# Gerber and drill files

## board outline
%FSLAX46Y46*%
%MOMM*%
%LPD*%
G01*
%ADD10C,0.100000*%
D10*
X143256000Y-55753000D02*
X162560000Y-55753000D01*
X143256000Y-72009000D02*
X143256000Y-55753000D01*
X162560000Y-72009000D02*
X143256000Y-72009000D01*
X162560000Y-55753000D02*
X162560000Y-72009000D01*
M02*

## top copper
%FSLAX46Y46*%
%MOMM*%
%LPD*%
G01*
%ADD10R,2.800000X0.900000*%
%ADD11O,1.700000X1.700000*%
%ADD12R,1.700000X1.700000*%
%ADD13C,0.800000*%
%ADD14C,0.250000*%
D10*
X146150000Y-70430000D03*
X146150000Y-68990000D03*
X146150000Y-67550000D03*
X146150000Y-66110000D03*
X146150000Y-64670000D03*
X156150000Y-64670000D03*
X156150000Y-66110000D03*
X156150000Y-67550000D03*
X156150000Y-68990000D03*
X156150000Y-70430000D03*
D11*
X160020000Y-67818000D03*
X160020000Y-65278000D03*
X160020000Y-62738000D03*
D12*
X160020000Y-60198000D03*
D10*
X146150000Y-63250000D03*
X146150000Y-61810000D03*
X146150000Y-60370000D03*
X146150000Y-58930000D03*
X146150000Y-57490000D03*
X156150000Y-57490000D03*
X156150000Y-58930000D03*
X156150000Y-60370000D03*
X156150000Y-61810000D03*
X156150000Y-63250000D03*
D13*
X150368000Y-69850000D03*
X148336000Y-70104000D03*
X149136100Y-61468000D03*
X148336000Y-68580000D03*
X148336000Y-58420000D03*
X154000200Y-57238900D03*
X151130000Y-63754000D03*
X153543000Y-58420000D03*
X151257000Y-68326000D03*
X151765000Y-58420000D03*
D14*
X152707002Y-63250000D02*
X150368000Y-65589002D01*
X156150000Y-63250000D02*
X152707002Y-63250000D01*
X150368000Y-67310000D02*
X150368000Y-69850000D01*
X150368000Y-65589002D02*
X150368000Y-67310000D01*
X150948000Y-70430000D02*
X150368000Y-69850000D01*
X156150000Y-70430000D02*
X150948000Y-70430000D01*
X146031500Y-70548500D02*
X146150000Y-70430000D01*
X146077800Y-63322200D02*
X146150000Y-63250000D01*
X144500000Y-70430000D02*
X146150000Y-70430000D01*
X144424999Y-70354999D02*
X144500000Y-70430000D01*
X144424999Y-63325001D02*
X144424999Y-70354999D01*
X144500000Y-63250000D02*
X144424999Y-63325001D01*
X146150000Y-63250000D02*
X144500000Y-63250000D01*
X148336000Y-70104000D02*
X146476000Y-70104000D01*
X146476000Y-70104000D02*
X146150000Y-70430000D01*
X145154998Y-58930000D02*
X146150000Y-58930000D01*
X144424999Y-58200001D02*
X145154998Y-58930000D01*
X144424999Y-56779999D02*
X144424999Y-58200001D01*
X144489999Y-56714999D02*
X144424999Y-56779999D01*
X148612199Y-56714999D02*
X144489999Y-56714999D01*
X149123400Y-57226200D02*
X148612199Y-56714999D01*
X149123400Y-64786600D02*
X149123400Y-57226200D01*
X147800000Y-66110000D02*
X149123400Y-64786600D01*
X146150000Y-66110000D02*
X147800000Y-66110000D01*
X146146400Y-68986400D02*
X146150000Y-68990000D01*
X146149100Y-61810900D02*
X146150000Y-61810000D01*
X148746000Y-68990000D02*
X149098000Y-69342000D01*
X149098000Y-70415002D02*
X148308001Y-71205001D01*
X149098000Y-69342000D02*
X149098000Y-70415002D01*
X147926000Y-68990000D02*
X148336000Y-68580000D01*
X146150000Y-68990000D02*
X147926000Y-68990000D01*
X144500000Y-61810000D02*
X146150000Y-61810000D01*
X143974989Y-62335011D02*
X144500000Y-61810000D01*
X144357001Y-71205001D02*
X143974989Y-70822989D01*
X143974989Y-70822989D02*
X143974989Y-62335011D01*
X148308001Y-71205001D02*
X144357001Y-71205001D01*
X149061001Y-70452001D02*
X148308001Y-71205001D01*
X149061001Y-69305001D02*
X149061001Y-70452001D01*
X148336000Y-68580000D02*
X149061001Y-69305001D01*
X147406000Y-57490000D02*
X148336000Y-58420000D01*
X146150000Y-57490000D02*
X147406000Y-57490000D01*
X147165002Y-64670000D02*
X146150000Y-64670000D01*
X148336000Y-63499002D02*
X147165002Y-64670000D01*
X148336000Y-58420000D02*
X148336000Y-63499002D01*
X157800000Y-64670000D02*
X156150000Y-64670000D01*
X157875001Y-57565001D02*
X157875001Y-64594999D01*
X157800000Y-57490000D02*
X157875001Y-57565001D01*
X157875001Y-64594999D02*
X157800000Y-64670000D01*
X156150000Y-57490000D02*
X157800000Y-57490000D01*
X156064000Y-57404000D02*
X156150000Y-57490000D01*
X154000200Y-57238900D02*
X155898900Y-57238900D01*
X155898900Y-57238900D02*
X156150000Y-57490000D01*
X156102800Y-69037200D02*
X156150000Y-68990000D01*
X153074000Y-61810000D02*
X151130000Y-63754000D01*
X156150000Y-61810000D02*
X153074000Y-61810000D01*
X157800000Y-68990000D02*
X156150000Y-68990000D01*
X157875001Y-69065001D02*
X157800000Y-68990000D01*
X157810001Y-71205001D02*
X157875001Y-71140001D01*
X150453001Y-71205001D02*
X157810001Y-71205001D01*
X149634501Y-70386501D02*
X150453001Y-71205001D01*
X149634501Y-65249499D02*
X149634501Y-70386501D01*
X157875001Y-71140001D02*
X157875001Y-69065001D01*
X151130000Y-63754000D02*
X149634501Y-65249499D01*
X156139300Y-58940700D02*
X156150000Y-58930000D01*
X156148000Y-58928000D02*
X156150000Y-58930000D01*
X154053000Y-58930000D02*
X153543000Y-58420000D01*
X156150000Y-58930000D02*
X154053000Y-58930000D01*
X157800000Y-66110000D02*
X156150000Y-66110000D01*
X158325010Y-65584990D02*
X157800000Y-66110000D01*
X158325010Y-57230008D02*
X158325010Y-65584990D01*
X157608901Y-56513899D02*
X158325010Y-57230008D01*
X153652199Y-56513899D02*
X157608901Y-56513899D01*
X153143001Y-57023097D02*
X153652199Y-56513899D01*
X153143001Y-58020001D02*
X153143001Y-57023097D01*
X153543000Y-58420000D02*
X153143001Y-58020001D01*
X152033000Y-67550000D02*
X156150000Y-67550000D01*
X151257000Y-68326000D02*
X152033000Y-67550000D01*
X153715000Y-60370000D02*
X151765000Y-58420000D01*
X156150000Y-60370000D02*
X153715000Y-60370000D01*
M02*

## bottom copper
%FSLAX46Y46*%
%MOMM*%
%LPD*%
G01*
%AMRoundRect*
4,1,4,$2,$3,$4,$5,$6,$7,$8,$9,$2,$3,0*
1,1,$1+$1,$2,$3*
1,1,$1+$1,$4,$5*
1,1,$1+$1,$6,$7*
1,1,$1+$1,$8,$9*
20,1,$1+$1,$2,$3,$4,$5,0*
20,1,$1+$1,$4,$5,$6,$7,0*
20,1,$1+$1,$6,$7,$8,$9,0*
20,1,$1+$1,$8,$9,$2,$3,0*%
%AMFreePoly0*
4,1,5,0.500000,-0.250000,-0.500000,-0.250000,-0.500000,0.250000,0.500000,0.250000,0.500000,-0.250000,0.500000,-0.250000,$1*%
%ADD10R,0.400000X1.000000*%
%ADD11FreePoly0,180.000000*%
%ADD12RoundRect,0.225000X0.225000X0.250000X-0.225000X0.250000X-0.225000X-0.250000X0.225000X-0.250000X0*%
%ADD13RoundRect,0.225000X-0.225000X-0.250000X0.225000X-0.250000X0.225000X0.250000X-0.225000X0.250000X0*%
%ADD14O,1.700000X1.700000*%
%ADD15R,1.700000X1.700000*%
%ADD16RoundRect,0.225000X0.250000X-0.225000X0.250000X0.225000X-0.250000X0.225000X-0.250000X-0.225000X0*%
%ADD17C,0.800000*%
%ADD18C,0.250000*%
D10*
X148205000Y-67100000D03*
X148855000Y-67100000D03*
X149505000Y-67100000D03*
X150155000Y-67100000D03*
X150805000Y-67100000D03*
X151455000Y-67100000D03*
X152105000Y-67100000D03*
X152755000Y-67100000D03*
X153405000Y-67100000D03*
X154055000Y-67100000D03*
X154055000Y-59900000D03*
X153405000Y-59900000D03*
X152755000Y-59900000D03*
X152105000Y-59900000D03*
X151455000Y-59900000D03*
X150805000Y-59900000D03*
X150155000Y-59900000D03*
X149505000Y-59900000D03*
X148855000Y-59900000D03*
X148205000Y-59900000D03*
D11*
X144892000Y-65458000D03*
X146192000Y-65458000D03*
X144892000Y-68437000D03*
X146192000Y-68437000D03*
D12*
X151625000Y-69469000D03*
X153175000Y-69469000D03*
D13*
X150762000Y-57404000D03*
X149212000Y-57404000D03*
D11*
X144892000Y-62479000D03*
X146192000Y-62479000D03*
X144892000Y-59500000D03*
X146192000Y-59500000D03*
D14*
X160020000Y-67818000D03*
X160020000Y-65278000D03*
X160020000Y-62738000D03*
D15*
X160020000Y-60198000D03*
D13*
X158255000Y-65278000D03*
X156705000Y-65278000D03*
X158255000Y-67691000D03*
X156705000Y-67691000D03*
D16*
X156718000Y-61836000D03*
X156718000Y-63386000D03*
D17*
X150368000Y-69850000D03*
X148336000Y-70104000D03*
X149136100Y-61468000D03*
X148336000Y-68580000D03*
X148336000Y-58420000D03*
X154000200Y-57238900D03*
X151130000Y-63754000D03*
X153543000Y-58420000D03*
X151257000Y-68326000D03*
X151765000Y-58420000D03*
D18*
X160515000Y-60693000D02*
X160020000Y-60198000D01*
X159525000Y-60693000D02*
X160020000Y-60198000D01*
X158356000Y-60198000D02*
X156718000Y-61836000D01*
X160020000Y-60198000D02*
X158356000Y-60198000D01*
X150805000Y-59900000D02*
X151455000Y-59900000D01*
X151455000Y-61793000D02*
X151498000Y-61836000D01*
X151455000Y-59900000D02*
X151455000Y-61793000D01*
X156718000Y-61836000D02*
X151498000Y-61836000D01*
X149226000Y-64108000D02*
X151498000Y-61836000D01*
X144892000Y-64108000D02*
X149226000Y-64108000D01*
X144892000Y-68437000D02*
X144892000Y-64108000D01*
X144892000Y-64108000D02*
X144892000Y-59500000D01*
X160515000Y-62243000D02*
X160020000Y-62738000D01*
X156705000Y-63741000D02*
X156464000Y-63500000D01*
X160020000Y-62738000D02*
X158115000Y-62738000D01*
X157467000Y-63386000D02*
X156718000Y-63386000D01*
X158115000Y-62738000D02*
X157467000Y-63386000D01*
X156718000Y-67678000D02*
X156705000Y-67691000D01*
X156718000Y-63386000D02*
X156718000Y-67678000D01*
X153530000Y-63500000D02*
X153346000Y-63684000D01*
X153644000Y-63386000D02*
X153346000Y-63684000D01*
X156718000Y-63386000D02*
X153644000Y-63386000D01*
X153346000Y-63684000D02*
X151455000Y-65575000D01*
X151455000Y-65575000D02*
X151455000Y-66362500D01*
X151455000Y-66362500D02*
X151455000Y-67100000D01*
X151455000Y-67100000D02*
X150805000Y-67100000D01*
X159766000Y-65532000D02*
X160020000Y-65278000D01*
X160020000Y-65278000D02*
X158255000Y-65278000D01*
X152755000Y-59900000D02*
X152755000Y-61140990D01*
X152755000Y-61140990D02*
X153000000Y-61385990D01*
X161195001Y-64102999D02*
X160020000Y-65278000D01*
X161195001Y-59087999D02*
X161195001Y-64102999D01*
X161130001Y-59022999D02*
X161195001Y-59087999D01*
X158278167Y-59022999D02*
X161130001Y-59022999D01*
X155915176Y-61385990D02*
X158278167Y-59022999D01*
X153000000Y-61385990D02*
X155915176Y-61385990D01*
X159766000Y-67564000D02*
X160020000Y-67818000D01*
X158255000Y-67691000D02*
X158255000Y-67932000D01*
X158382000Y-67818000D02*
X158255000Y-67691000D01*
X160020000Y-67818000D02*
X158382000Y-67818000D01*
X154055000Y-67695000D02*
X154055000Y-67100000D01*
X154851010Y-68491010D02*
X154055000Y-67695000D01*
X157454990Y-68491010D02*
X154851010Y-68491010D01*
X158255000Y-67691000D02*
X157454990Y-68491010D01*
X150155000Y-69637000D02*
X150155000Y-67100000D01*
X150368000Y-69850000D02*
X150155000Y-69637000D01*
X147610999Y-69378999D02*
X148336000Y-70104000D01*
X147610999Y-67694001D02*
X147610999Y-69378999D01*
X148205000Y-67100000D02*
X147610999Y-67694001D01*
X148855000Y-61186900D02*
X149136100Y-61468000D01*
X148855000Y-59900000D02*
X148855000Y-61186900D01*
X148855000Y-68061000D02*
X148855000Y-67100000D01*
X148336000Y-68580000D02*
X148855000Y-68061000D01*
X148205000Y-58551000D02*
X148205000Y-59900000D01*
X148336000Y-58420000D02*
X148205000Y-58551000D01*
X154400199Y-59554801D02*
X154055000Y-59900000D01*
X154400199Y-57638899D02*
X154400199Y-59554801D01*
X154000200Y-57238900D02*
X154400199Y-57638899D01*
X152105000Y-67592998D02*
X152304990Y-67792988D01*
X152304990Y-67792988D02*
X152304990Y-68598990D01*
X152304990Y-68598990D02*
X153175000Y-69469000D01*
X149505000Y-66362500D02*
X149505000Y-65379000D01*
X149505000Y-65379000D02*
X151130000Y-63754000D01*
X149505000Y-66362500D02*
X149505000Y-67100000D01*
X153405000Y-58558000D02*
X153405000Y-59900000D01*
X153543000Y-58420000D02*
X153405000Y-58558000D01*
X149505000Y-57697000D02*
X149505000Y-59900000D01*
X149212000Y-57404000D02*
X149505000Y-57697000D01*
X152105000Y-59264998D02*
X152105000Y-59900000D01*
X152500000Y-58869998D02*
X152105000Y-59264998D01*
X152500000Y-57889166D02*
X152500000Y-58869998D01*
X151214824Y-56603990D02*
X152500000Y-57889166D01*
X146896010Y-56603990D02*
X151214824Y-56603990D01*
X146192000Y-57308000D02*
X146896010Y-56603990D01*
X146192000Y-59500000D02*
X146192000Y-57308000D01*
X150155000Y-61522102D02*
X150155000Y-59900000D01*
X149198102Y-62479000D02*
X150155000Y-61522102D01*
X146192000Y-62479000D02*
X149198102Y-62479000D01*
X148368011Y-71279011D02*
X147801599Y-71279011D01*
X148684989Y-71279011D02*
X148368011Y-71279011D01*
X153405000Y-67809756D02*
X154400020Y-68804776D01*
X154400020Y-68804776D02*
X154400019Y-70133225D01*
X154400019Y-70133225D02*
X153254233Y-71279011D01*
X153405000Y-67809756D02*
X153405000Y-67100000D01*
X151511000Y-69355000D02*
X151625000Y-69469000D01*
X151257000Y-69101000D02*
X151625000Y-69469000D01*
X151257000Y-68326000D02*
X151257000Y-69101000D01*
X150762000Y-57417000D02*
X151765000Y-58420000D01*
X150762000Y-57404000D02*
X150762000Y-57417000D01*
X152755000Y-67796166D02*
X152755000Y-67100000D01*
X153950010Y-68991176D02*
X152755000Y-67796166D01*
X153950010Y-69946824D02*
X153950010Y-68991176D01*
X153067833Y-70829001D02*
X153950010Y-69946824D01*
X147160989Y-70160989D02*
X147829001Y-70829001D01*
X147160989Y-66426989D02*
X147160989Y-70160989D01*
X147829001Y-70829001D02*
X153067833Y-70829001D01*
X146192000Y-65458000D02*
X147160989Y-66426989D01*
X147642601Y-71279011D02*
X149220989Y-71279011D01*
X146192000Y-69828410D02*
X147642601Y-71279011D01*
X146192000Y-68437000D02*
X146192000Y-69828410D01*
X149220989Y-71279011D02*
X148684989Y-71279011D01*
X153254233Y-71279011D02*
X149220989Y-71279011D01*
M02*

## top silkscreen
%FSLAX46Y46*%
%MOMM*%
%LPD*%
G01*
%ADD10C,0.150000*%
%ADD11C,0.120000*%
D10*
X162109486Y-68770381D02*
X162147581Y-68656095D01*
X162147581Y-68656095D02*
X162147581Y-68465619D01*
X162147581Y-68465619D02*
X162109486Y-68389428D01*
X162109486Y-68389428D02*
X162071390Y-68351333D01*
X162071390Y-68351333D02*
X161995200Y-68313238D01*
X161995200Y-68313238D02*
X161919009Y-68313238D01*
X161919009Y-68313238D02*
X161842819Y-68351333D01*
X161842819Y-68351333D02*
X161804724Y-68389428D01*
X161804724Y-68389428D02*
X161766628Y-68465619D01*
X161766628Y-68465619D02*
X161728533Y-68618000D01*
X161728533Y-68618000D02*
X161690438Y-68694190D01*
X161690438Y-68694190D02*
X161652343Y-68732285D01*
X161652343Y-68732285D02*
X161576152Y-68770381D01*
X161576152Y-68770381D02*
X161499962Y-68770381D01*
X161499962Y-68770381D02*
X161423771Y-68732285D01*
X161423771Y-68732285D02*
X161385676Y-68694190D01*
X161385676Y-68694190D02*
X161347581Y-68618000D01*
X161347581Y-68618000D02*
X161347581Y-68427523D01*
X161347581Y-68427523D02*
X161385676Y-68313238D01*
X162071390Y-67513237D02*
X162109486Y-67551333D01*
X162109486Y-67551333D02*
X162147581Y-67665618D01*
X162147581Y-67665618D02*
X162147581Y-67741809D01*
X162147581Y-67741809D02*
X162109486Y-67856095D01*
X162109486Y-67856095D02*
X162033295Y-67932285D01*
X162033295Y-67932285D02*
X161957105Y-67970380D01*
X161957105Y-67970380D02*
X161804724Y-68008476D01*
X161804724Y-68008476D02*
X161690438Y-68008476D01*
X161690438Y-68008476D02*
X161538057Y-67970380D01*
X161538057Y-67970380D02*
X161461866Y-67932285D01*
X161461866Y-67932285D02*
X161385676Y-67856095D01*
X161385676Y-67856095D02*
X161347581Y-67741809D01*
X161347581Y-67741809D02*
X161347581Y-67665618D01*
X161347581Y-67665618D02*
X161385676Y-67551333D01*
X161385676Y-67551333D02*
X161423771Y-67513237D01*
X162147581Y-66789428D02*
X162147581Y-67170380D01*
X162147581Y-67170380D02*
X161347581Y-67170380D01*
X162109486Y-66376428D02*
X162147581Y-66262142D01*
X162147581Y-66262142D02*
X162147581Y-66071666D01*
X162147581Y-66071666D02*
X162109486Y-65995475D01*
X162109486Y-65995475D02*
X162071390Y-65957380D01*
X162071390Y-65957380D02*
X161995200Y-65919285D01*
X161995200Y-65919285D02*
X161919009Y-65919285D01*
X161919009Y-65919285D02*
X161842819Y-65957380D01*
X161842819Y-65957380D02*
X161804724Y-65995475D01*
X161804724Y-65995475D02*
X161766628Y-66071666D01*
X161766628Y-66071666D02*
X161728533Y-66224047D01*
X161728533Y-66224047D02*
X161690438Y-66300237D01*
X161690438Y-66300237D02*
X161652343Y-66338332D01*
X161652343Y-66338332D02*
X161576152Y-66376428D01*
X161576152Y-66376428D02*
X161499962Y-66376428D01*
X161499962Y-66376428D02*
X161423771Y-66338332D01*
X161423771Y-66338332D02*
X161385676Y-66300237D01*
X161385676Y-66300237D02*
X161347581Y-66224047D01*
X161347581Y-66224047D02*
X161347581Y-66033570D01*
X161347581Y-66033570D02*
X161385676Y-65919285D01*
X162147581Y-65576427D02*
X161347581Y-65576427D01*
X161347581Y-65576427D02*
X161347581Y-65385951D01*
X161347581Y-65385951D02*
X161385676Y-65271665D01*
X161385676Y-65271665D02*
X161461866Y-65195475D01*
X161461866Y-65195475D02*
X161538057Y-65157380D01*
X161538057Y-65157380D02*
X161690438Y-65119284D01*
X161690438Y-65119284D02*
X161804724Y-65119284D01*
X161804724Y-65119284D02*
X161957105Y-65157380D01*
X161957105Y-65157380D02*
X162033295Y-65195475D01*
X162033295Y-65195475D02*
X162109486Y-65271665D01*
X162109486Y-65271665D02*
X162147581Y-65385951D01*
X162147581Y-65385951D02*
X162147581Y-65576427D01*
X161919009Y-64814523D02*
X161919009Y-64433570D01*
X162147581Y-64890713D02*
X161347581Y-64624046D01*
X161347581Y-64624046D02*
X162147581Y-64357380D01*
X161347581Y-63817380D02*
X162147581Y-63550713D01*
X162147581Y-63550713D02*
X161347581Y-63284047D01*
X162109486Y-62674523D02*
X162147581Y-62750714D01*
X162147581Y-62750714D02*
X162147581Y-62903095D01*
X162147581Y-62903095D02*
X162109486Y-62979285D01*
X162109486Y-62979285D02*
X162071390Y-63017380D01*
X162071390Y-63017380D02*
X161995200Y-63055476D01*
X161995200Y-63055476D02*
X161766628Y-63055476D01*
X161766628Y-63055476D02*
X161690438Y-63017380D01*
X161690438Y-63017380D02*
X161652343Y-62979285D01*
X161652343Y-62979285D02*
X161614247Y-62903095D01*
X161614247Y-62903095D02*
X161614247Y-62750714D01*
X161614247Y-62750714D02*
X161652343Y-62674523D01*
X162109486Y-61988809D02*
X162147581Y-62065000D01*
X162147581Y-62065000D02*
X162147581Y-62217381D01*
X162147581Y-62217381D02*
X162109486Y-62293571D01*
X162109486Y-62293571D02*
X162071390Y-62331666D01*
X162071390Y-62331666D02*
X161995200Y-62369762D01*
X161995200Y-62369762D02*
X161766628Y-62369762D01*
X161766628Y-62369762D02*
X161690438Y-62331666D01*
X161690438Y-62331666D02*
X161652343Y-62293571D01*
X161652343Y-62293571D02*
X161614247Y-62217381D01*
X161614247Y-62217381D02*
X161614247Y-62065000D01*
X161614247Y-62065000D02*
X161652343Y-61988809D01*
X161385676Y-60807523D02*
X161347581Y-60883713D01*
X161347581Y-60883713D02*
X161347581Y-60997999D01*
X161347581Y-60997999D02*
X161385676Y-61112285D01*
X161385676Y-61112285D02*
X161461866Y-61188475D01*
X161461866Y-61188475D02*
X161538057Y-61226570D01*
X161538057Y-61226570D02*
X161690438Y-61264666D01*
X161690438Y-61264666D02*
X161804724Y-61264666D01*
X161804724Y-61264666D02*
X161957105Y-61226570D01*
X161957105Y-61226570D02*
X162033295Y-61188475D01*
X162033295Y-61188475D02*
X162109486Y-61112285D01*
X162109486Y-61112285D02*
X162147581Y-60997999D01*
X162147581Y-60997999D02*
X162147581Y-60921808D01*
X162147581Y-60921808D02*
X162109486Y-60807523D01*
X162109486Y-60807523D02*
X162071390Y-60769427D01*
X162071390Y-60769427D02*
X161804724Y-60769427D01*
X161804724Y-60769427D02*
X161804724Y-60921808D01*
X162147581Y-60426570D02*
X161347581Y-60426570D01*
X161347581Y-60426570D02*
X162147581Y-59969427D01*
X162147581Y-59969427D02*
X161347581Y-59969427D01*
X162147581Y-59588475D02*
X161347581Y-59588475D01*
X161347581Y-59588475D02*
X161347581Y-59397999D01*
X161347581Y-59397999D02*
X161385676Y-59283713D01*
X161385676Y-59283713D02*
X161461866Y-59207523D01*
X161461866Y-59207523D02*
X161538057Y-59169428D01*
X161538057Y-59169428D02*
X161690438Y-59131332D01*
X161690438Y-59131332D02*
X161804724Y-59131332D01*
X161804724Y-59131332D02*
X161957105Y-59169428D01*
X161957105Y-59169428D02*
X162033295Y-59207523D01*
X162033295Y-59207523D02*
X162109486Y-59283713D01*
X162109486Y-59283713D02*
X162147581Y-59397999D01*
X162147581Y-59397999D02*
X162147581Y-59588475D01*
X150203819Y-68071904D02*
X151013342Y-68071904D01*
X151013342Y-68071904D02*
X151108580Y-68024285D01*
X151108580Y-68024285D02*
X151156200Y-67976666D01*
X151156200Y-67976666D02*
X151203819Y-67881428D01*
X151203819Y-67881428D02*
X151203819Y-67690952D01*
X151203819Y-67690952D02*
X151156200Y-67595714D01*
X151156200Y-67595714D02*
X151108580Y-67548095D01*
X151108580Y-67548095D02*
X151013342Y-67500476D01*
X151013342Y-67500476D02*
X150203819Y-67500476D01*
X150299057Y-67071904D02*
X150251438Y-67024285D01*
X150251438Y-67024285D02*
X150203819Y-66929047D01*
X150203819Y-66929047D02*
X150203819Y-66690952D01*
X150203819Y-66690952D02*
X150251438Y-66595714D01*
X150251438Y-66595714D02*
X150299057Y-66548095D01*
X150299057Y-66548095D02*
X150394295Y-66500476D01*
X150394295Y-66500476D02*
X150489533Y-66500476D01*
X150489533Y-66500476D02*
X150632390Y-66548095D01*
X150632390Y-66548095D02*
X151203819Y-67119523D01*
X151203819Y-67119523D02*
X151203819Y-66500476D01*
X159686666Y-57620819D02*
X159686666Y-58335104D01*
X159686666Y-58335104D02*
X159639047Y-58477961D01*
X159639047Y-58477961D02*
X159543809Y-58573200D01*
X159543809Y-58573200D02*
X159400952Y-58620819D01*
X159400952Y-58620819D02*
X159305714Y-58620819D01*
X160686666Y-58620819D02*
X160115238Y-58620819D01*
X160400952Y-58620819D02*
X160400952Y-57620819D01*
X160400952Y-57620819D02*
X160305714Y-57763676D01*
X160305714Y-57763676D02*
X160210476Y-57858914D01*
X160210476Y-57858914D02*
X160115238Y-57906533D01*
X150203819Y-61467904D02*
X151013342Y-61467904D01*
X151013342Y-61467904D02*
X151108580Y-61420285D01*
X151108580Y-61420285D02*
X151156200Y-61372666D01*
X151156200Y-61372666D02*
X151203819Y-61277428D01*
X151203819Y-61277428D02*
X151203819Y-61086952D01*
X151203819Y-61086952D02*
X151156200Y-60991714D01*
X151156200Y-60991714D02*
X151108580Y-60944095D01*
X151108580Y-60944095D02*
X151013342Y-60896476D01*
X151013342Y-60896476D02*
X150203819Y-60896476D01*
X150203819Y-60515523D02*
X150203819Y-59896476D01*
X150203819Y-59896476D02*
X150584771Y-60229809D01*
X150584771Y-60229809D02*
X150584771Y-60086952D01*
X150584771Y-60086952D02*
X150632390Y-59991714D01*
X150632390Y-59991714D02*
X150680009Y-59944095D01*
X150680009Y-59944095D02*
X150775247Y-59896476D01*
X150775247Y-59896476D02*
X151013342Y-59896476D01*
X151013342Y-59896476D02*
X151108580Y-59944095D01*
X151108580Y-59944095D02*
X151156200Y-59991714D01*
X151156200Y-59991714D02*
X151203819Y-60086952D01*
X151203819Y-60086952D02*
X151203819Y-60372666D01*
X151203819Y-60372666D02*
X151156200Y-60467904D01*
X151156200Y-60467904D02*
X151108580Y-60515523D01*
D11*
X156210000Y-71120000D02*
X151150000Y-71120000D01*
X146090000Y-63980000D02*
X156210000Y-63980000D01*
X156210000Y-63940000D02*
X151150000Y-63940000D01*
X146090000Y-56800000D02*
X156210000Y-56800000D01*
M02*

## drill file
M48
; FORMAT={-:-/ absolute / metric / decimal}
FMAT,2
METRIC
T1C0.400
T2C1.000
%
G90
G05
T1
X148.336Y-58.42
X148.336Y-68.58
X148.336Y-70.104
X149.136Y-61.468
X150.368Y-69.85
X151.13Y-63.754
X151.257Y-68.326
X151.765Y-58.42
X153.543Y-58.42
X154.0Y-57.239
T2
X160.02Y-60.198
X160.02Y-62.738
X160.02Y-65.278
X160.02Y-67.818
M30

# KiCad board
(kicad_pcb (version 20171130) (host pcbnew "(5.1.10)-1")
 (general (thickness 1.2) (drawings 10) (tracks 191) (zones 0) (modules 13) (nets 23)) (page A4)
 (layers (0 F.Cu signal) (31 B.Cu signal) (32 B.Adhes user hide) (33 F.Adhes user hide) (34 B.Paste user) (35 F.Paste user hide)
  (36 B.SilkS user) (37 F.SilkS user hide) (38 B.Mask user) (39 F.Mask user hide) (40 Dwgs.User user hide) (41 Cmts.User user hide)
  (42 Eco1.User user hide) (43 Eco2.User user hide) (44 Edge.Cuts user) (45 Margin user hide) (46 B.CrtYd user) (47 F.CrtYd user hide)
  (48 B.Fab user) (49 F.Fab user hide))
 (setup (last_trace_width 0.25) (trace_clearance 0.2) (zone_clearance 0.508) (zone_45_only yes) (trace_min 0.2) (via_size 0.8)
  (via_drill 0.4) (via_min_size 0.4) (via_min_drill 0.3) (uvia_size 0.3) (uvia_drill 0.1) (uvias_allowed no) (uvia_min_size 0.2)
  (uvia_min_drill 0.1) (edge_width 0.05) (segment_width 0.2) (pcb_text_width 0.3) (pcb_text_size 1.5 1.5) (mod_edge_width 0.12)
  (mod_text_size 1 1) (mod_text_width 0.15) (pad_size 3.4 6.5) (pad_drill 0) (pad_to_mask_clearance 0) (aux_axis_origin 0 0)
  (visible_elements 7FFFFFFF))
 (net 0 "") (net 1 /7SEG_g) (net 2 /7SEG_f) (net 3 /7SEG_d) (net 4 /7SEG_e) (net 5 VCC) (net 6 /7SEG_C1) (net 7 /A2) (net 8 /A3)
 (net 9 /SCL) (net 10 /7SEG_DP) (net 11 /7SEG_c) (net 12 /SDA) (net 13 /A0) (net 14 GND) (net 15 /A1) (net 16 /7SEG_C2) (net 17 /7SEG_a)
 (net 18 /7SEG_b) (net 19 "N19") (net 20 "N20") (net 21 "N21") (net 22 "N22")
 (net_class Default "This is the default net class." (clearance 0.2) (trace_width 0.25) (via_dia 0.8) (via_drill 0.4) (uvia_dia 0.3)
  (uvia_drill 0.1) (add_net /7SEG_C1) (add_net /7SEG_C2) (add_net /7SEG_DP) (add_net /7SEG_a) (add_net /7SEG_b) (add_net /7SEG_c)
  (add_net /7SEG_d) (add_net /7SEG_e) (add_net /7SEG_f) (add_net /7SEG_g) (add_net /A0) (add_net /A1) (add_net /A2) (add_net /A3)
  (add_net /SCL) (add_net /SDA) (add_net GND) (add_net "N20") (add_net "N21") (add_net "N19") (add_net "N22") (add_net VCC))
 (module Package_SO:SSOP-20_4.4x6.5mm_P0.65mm (layer B.Cu) (at 151.13 63.5 270)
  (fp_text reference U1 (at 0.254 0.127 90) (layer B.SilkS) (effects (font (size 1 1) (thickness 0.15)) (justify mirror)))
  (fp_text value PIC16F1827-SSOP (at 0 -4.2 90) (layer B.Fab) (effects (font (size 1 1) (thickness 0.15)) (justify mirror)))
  (pad 20 smd rect (at 3.6 2.925 270) (size 1 0.4) (layers B.Cu B.Paste B.Mask) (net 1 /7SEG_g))
  (pad 19 smd rect (at 3.6 2.275 270) (size 1 0.4) (layers B.Cu B.Paste B.Mask) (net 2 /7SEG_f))
  (pad 18 smd rect (at 3.6 1.625 270) (size 1 0.4) (layers B.Cu B.Paste B.Mask) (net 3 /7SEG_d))
  (pad 17 smd rect (at 3.6 0.975 270) (size 1 0.4) (layers B.Cu B.Paste B.Mask) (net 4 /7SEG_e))
  (pad 16 smd rect (at 3.6 0.325 270) (size 1 0.4) (layers B.Cu B.Paste B.Mask) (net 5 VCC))
  (pad 15 smd rect (at 3.6 -0.325 270) (size 1 0.4) (layers B.Cu B.Paste B.Mask) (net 5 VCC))
  (pad 14 smd rect (at 3.6 -0.975 270) (size 1 0.4) (layers B.Cu B.Paste B.Mask) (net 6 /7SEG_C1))
  (pad 13 smd rect (at 3.6 -1.625 270) (size 1 0.4) (layers B.Cu B.Paste B.Mask) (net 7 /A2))
  (pad 12 smd rect (at 3.6 -2.275 270) (size 1 0.4) (layers B.Cu B.Paste B.Mask) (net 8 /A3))
  (pad 11 smd rect (at 3.6 -2.925 270) (size 1 0.4) (layers B.Cu B.Paste B.Mask) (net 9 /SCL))
  (pad 10 smd rect (at -3.6 -2.925 270) (size 1 0.4) (layers B.Cu B.Paste B.Mask) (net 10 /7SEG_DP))
  (pad 9 smd rect (at -3.6 -2.275 270) (size 1 0.4) (layers B.Cu B.Paste B.Mask) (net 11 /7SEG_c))
  (pad 8 smd rect (at -3.6 -1.625 270) (size 1 0.4) (layers B.Cu B.Paste B.Mask) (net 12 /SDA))
  (pad 7 smd rect (at -3.6 -0.975 270) (size 1 0.4) (layers B.Cu B.Paste B.Mask) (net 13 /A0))
  (pad 6 smd rect (at -3.6 -0.325 270) (size 1 0.4) (layers B.Cu B.Paste B.Mask) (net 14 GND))
  (pad 5 smd rect (at -3.6 0.325 270) (size 1 0.4) (layers B.Cu B.Paste B.Mask) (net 14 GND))
  (pad 4 smd rect (at -3.6 0.975 270) (size 1 0.4) (layers B.Cu B.Paste B.Mask) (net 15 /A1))
  (pad 3 smd rect (at -3.6 1.625 270) (size 1 0.4) (layers B.Cu B.Paste B.Mask) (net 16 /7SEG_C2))
  (pad 2 smd rect (at -3.6 2.275 270) (size 1 0.4) (layers B.Cu B.Paste B.Mask) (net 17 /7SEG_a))
  (pad 1 smd rect (at -3.6 2.925 270) (size 1 0.4) (layers B.Cu B.Paste B.Mask) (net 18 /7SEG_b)))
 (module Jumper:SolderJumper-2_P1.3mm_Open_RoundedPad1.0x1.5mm (layer B.Cu) (at 145.542 65.458 180)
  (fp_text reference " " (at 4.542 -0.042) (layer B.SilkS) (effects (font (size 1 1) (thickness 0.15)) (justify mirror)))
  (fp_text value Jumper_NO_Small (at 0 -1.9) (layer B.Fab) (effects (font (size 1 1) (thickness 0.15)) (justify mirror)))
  (pad 2 smd custom (at 0.65 0 180) (size 1 0.5) (layers B.Cu B.Mask) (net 14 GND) (zone_connect 2)
   (options (clearance outline) (anchor rect)) (primitives))
  (pad 1 smd custom (at -0.65 0 180) (size 1 0.5) (layers B.Cu B.Mask) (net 7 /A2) (zone_connect 2)
   (options (clearance outline) (anchor rect)) (primitives)))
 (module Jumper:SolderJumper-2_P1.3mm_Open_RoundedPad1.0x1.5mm (layer B.Cu) (at 145.542 68.437 180)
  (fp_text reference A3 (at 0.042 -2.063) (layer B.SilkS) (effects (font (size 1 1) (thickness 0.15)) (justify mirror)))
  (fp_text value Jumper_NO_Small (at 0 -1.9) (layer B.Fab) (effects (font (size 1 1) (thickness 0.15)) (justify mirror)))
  (pad 2 smd custom (at 0.65 0 180) (size 1 0.5) (layers B.Cu B.Mask) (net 14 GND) (zone_connect 2)
   (options (clearance outline) (anchor rect)) (primitives))
  (pad 1 smd custom (at -0.65 0 180) (size 1 0.5) (layers B.Cu B.Mask) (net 8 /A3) (zone_connect 2)
   (options (clearance outline) (anchor rect)) (primitives)))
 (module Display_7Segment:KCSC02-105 (layer F.Cu) (at 151.15 67.55 180)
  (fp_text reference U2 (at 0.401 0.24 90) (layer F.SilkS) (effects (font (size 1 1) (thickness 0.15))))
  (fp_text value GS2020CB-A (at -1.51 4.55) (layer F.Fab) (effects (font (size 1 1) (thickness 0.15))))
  (fp_line (start -5.06 -3.57) (end 0 -3.57) (layer F.SilkS) (width 0.12))
  (fp_line (start 5.06 3.57) (end -5.06 3.57) (layer F.SilkS) (width 0.12))
  (pad 10 smd rect (at 5 -2.88 180) (size 2.8 0.9) (layers F.Cu F.Paste F.Mask) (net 1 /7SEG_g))
  (pad 9 smd rect (at 5 -1.44 180) (size 2.8 0.9) (layers F.Cu F.Paste F.Mask) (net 2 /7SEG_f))
  (pad 8 smd rect (at 5 0 180) (size 2.8 0.9) (layers F.Cu F.Paste F.Mask) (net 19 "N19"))
  (pad 7 smd rect (at 5 1.44 180) (size 2.8 0.9) (layers F.Cu F.Paste F.Mask) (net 17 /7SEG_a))
  (pad 6 smd rect (at 5 2.88 180) (size 2.8 0.9) (layers F.Cu F.Paste F.Mask) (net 18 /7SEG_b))
  (pad 5 smd rect (at -5 2.88 180) (size 2.8 0.9) (layers F.Cu F.Paste F.Mask) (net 10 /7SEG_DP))
  (pad 4 smd rect (at -5 1.44 180) (size 2.8 0.9) (layers F.Cu F.Paste F.Mask) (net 11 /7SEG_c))
  (pad 3 smd rect (at -5 0 180) (size 2.8 0.9) (layers F.Cu F.Paste F.Mask) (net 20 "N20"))
  (pad 2 smd rect (at -5 -1.44 180) (size 2.8 0.9) (layers F.Cu F.Paste F.Mask) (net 3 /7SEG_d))
  (pad 1 smd rect (at -5 -2.88 180) (size 2.8 0.9) (layers F.Cu F.Paste F.Mask) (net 4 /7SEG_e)))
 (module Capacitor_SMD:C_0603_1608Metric (layer B.Cu) (at 152.4 69.469 180)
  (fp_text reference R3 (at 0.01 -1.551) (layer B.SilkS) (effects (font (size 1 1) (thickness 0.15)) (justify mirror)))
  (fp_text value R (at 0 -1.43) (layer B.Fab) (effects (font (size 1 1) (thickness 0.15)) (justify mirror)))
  (pad 2 smd roundrect (at 0.775 0 180) (size 0.9 0.95) (layers B.Cu B.Paste B.Mask) (roundrect_rratio 0.25) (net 20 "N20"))
  (pad 1 smd roundrect (at -0.775 0 180) (size 0.9 0.95) (layers B.Cu B.Paste B.Mask) (roundrect_rratio 0.25) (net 6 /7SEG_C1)))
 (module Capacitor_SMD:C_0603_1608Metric (layer B.Cu) (at 149.987 57.404)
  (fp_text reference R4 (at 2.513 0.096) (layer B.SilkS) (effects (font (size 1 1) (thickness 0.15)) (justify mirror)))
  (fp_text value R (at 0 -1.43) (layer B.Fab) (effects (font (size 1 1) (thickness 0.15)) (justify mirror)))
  (pad 2 smd roundrect (at 0.775 0) (size 0.9 0.95) (layers B.Cu B.Paste B.Mask) (roundrect_rratio 0.25) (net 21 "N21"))
  (pad 1 smd roundrect (at -0.775 0) (size 0.9 0.95) (layers B.Cu B.Paste B.Mask) (roundrect_rratio 0.25) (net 16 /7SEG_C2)))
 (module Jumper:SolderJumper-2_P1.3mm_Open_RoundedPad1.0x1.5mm (layer B.Cu) (at 145.542 62.479 180)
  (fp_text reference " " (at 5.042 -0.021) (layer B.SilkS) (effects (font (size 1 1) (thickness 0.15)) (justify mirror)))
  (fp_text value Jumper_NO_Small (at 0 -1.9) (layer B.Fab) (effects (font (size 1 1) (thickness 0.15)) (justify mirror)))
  (pad 2 smd custom (at 0.65 0 180) (size 1 0.5) (layers B.Cu B.Mask) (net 14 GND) (zone_connect 2)
   (options (clearance outline) (anchor rect)) (primitives))
  (pad 1 smd custom (at -0.65 0 180) (size 1 0.5) (layers B.Cu B.Mask) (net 15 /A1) (zone_connect 2)
   (options (clearance outline) (anchor rect)) (primitives)))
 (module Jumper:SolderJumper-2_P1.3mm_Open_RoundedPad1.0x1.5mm (layer B.Cu) (at 145.542 59.5 180)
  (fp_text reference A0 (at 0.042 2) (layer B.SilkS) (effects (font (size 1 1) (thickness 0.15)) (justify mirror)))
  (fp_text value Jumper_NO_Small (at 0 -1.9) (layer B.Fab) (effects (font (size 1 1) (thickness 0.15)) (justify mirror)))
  (pad 2 smd custom (at 0.65 0 180) (size 1 0.5) (layers B.Cu B.Mask) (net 14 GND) (zone_connect 2)
   (options (clearance outline) (anchor rect)) (primitives))
  (pad 1 smd custom (at -0.65 0 180) (size 1 0.5) (layers B.Cu B.Mask) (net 13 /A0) (zone_connect 2)
   (options (clearance outline) (anchor rect)) (primitives)))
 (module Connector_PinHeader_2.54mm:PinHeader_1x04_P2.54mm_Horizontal (layer F.Cu) (at 160.02 60.198)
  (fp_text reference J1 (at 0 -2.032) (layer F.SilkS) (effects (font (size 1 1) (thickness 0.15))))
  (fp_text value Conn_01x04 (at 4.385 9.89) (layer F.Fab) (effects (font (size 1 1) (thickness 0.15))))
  (pad 4 thru_hole oval (at 0 7.62) (size 1.7 1.7) (drill 1) (layers *.Cu *.Mask) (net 9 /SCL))
  (pad 3 thru_hole oval (at 0 5.08) (size 1.7 1.7) (drill 1) (layers *.Cu *.Mask) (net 12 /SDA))
  (pad 2 thru_hole oval (at 0 2.54) (size 1.7 1.7) (drill 1) (layers *.Cu *.Mask) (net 5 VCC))
  (pad 1 thru_hole rect (at 0 0) (size 1.7 1.7) (drill 1) (layers *.Cu *.Mask) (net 14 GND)))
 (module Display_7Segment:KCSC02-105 (layer F.Cu) (at 151.15 60.37 180)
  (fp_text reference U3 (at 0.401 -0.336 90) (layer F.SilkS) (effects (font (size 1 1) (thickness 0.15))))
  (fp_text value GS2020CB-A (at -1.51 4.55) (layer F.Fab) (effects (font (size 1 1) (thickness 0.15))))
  (fp_line (start -5.06 -3.57) (end 0 -3.57) (layer F.SilkS) (width 0.12))
  (fp_line (start 5.06 3.57) (end -5.06 3.57) (layer F.SilkS) (width 0.12))
  (pad 10 smd rect (at 5 -2.88 180) (size 2.8 0.9) (layers F.Cu F.Paste F.Mask) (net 1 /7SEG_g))
  (pad 9 smd rect (at 5 -1.44 180) (size 2.8 0.9) (layers F.Cu F.Paste F.Mask) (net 2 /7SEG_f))
  (pad 8 smd rect (at 5 0 180) (size 2.8 0.9) (layers F.Cu F.Paste F.Mask) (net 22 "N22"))
  (pad 7 smd rect (at 5 1.44 180) (size 2.8 0.9) (layers F.Cu F.Paste F.Mask) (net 17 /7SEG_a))
  (pad 6 smd rect (at 5 2.88 180) (size 2.8 0.9) (layers F.Cu F.Paste F.Mask) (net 18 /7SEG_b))
  (pad 5 smd rect (at -5 2.88 180) (size 2.8 0.9) (layers F.Cu F.Paste F.Mask) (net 10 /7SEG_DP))
  (pad 4 smd rect (at -5 1.44 180) (size 2.8 0.9) (layers F.Cu F.Paste F.Mask) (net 11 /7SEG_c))
  (pad 3 smd rect (at -5 0 180) (size 2.8 0.9) (layers F.Cu F.Paste F.Mask) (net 21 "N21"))
  (pad 2 smd rect (at -5 -1.44 180) (size 2.8 0.9) (layers F.Cu F.Paste F.Mask) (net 3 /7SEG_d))
  (pad 1 smd rect (at -5 -2.88 180) (size 2.8 0.9) (layers F.Cu F.Paste F.Mask) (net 4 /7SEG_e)))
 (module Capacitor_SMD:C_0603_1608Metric (layer B.Cu) (at 157.48 65.278)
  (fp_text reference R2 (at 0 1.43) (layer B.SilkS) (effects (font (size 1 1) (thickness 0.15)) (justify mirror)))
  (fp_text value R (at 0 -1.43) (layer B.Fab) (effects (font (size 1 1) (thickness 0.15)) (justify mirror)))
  (pad 2 smd roundrect (at 0.775 0) (size 0.9 0.95) (layers B.Cu B.Paste B.Mask) (roundrect_rratio 0.25) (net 12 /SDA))
  (pad 1 smd roundrect (at -0.775 0) (size 0.9 0.95) (layers B.Cu B.Paste B.Mask) (roundrect_rratio 0.25) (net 5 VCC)))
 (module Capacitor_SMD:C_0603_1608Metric (layer B.Cu) (at 157.48 67.691)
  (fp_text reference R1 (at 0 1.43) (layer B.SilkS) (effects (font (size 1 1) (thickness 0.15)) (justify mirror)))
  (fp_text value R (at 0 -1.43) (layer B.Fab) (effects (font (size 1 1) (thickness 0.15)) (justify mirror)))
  (pad 2 smd roundrect (at 0.775 0) (size 0.9 0.95) (layers B.Cu B.Paste B.Mask) (roundrect_rratio 0.25) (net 9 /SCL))
  (pad 1 smd roundrect (at -0.775 0) (size 0.9 0.95) (layers B.Cu B.Paste B.Mask) (roundrect_rratio 0.25) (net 5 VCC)))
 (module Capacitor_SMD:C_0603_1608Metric (layer B.Cu) (at 156.718 62.611 90)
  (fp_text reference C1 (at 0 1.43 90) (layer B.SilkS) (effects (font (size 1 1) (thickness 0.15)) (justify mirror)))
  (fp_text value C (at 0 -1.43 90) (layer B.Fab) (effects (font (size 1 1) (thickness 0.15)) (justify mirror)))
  (pad 2 smd roundrect (at 0.775 0 90) (size 0.9 0.95) (layers B.Cu B.Paste B.Mask) (roundrect_rratio 0.25) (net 14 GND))
  (pad 1 smd roundrect (at -0.775 0 90) (size 0.9 0.95) (layers B.Cu B.Paste B.Mask) (roundrect_rratio 0.25) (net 5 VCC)))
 (gr_line (start 143.256 55.753) (end 162.56 55.753) (layer Edge.Cuts) (width 0.1))
 (gr_line (start 143.256 72.009) (end 143.256 55.753) (layer Edge.Cuts) (width 0.1))
 (gr_line (start 162.56 72.009) (end 143.256 72.009) (layer Edge.Cuts) (width 0.1))
 (gr_line (start 162.56 55.753) (end 162.56 72.009) (layer Edge.Cuts) (width 0.1))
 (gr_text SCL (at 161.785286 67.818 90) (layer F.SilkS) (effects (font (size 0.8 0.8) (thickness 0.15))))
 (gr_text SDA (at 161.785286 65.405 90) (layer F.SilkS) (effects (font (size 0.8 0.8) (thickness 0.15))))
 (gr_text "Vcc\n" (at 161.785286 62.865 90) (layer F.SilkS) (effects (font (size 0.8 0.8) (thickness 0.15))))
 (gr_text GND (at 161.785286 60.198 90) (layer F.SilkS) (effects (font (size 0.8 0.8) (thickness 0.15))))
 (segment (start 160.515 60.693) (end 160.02 60.198) (width 0.25) (layer B.Cu) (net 14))
 (segment (start 159.525 60.693) (end 160.02 60.198) (width 0.25) (layer B.Cu) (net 14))
 (segment (start 158.356 60.198) (end 156.718 61.836) (width 0.25) (layer B.Cu) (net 14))
 (segment (start 160.02 60.198) (end 158.356 60.198) (width 0.25) (layer B.Cu) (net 14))
 (segment (start 150.805 59.9) (end 151.455 59.9) (width 0.25) (layer B.Cu) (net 14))
 (segment (start 151.455 61.793) (end 151.498 61.836) (width 0.25) (layer B.Cu) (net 14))
 (segment (start 151.455 59.9) (end 151.455 61.793) (width 0.25) (layer B.Cu) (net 14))
 (segment (start 156.718 61.836) (end 151.498 61.836) (width 0.25) (layer B.Cu) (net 14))
 (segment (start 149.226 64.108) (end 151.498 61.836) (width 0.25) (layer B.Cu) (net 14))
 (segment (start 144.892 64.108) (end 149.226 64.108) (width 0.25) (layer B.Cu) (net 14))
 (segment (start 144.892 68.437) (end 144.892 64.108) (width 0.25) (layer B.Cu) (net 14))
 (segment (start 144.892 64.108) (end 144.892 59.5) (width 0.25) (layer B.Cu) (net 14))
 (segment (start 160.515 62.243) (end 160.02 62.738) (width 0.25) (layer B.Cu) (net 5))
 (segment (start 156.705 63.741) (end 156.464 63.5) (width 0.25) (layer B.Cu) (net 5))
 (segment (start 160.02 62.738) (end 158.115 62.738) (width 0.25) (layer B.Cu) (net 5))
 (segment (start 157.467 63.386) (end 156.718 63.386) (width 0.25) (layer B.Cu) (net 5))
 (segment (start 158.115 62.738) (end 157.467 63.386) (width 0.25) (layer B.Cu) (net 5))
 (segment (start 156.718 67.678) (end 156.705 67.691) (width 0.25) (layer B.Cu) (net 5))
 (segment (start 156.718 63.386) (end 156.718 67.678) (width 0.25) (layer B.Cu) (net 5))
 (segment (start 153.53 63.5) (end 153.346 63.684) (width 0.25) (layer B.Cu) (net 5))
 (segment (start 153.644 63.386) (end 153.346 63.684) (width 0.25) (layer B.Cu) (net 5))
 (segment (start 156.718 63.386) (end 153.644 63.386) (width 0.25) (layer B.Cu) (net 5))
 (segment (start 153.346 63.684) (end 151.455 65.575) (width 0.25) (layer B.Cu) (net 5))
 (segment (start 151.455 65.575) (end 151.455 66.3625) (width 0.25) (layer B.Cu) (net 5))
 (segment (start 151.455 66.3625) (end 151.455 67.1) (width 0.25) (layer B.Cu) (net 5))
 (segment (start 151.455 67.1) (end 150.805 67.1) (width 0.25) (layer B.Cu) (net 5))
 (segment (start 159.766 65.532) (end 160.02 65.278) (width 0.25) (layer B.Cu) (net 12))
 (segment (start 160.02 65.278) (end 158.255 65.278) (width 0.25) (layer B.Cu) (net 12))
 (segment (start 152.755 59.9) (end 152.755 61.14099) (width 0.25) (layer B.Cu) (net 12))
 (segment (start 152.755 61.14099) (end 153 61.38599) (width 0.25) (layer B.Cu) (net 12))
 (segment (start 161.195001 64.102999) (end 160.02 65.278) (width 0.25) (layer B.Cu) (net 12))
 (segment (start 161.195001 59.087999) (end 161.195001 64.102999) (width 0.25) (layer B.Cu) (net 12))
 (segment (start 161.130001 59.022999) (end 161.195001 59.087999) (width 0.25) (layer B.Cu) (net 12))
 (segment (start 158.278167 59.022999) (end 161.130001 59.022999) (width 0.25) (layer B.Cu) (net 12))
 (segment (start 155.915176 61.38599) (end 158.278167 59.022999) (width 0.25) (layer B.Cu) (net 12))
 (segment (start 153 61.38599) (end 155.915176 61.38599) (width 0.25) (layer B.Cu) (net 12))
 (segment (start 159.766 67.564) (end 160.02 67.818) (width 0.25) (layer B.Cu) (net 9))
 (segment (start 158.255 67.691) (end 158.255 67.932) (width 0.25) (layer B.Cu) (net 9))
 (segment (start 158.382 67.818) (end 158.255 67.691) (width 0.25) (layer B.Cu) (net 9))
 (segment (start 160.02 67.818) (end 158.382 67.818) (width 0.25) (layer B.Cu) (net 9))
 (segment (start 154.055 67.695) (end 154.055 67.1) (width 0.25) (layer B.Cu) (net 9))
 (segment (start 154.85101 68.49101) (end 154.055 67.695) (width 0.25) (layer B.Cu) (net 9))
 (segment (start 157.45499 68.49101) (end 154.85101 68.49101) (width 0.25) (layer B.Cu) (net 9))
 (segment (start 158.255 67.691) (end 157.45499 68.49101) (width 0.25) (layer B.Cu) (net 9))
 (segment (start 152.707002 63.25) (end 150.368 65.589002) (width 0.25) (layer F.Cu) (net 4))
 (segment (start 156.15 63.25) (end 152.707002 63.25) (width 0.25) (layer F.Cu) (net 4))
 (segment (start 150.368 67.31) (end 150.368 69.85) (width 0.25) (layer F.Cu) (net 4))
 (segment (start 150.368 65.589002) (end 150.368 67.31) (width 0.25) (layer F.Cu) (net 4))
 (segment (start 150.948 70.43) (end 150.368 69.85) (width 0.25) (layer F.Cu) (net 4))
 (segment (start 156.15 70.43) (end 150.948 70.43) (width 0.25) (layer F.Cu) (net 4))
 (via (at 150.368 69.85) (size 0.8) (drill 0.4) (layers F.Cu B.Cu) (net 4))
 (segment (start 150.155 69.637) (end 150.155 67.1) (width 0.25) (layer B.Cu) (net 4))
 (segment (start 150.368 69.85) (end 150.155 69.637) (width 0.25) (layer B.Cu) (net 4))
 (segment (start 146.0315 70.5485) (end 146.15 70.43) (width 0.25) (layer F.Cu) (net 1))
 (segment (start 146.0778 63.3222) (end 146.15 63.25) (width 0.25) (layer F.Cu) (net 1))
 (segment (start 144.5 70.43) (end 146.15 70.43) (width 0.25) (layer F.Cu) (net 1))
 (segment (start 144.424999 70.354999) (end 144.5 70.43) (width 0.25) (layer F.Cu) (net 1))
 (segment (start 144.424999 63.325001) (end 144.424999 70.354999) (width 0.25) (layer F.Cu) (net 1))
 (segment (start 144.5 63.25) (end 144.424999 63.325001) (width 0.25) (layer F.Cu) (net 1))
 (segment (start 146.15 63.25) (end 144.5 63.25) (width 0.25) (layer F.Cu) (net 1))
 (segment (start 148.336 70.104) (end 146.476 70.104) (width 0.25) (layer F.Cu) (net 1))
 (segment (start 146.476 70.104) (end 146.15 70.43) (width 0.25) (layer F.Cu) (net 1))
 (via (at 148.336 70.104) (size 0.8) (drill 0.4) (layers F.Cu B.Cu) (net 1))
 (segment (start 147.610999 69.378999) (end 148.336 70.104) (width 0.25) (layer B.Cu) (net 1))
 (segment (start 147.610999 67.694001) (end 147.610999 69.378999) (width 0.25) (layer B.Cu) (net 1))
 (segment (start 148.205 67.1) (end 147.610999 67.694001) (width 0.25) (layer B.Cu) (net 1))
 (via (at 149.1361 61.468) (size 0.8) (drill 0.4) (layers F.Cu B.Cu) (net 17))
 (segment (start 145.154998 58.93) (end 146.15 58.93) (width 0.25) (layer F.Cu) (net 17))
 (segment (start 144.424999 58.200001) (end 145.154998 58.93) (width 0.25) (layer F.Cu) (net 17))
 (segment (start 144.424999 56.779999) (end 144.424999 58.200001) (width 0.25) (layer F.Cu) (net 17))
 (segment (start 144.489999 56.714999) (end 144.424999 56.779999) (width 0.25) (layer F.Cu) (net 17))
 (segment (start 148.612199 56.714999) (end 144.489999 56.714999) (width 0.25) (layer F.Cu) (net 17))
 (segment (start 149.1234 57.2262) (end 148.612199 56.714999) (width 0.25) (layer F.Cu) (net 17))
 (segment (start 149.1234 64.7866) (end 149.1234 57.2262) (width 0.25) (layer F.Cu) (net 17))
 (segment (start 147.8 66.11) (end 149.1234 64.7866) (width 0.25) (layer F.Cu) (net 17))
 (segment (start 146.15 66.11) (end 147.8 66.11) (width 0.25) (layer F.Cu) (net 17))
 (segment (start 148.855 61.1869) (end 149.1361 61.468) (width 0.25) (layer B.Cu) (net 17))
 (segment (start 148.855 59.9) (end 148.855 61.1869) (width 0.25) (layer B.Cu) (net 17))
 (segment (start 146.1464 68.9864) (end 146.15 68.99) (width 0.25) (layer F.Cu) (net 2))
 (segment (start 146.1491 61.8109) (end 146.15 61.81) (width 0.25) (layer F.Cu) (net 2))
 (segment (start 148.746 68.99) (end 149.098 69.342) (width 0.25) (layer F.Cu) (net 2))
 (segment (start 149.098 70.415002) (end 148.308001 71.205001) (width 0.25) (layer F.Cu) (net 2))
 (segment (start 149.098 69.342) (end 149.098 70.415002) (width 0.25) (layer F.Cu) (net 2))
 (segment (start 147.926 68.99) (end 148.336 68.58) (width 0.25) (layer F.Cu) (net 2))
 (segment (start 146.15 68.99) (end 147.926 68.99) (width 0.25) (layer F.Cu) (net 2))
 (segment (start 144.5 61.81) (end 146.15 61.81) (width 0.25) (layer F.Cu) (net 2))
 (segment (start 143.974989 62.335011) (end 144.5 61.81) (width 0.25) (layer F.Cu) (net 2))
 (segment (start 144.357001 71.205001) (end 143.974989 70.822989) (width 0.25) (layer F.Cu) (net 2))
 (segment (start 143.974989 70.822989) (end 143.974989 62.335011) (width 0.25) (layer F.Cu) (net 2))
 (segment (start 148.308001 71.205001) (end 144.357001 71.205001) (width 0.25) (layer F.Cu) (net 2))
 (segment (start 149.061001 70.452001) (end 148.308001 71.205001) (width 0.25) (layer F.Cu) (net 2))
 (segment (start 149.061001 69.305001) (end 149.061001 70.452001) (width 0.25) (layer F.Cu) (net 2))
 (segment (start 148.336 68.58) (end 149.061001 69.305001) (width 0.25) (layer F.Cu) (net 2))
 (via (at 148.336 68.58) (size 0.8) (drill 0.4) (layers F.Cu B.Cu) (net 2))
 (segment (start 148.855 68.061) (end 148.855 67.1) (width 0.25) (layer B.Cu) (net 2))
 (segment (start 148.336 68.58) (end 148.855 68.061) (width 0.25) (layer B.Cu) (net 2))
 (via (at 148.336 58.42) (size 0.8) (drill 0.4) (layers F.Cu B.Cu) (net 18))
 (segment (start 147.406 57.49) (end 148.336 58.42) (width 0.25) (layer F.Cu) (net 18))
 (segment (start 146.15 57.49) (end 147.406 57.49) (width 0.25) (layer F.Cu) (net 18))
 (segment (start 147.165002 64.67) (end 146.15 64.67) (width 0.25) (layer F.Cu) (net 18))
 (segment (start 148.336 63.499002) (end 147.165002 64.67) (width 0.25) (layer F.Cu) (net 18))
 (segment (start 148.336 58.42) (end 148.336 63.499002) (width 0.25) (layer F.Cu) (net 18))
 (segment (start 148.205 58.551) (end 148.205 59.9) (width 0.25) (layer B.Cu) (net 18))
 (segment (start 148.336 58.42) (end 148.205 58.551) (width 0.25) (layer B.Cu) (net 18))
 (segment (start 157.8 64.67) (end 156.15 64.67) (width 0.25) (layer F.Cu) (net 10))
 (segment (start 157.875001 57.565001) (end 157.875001 64.594999) (width 0.25) (layer F.Cu) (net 10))
 (segment (start 157.8 57.49) (end 157.875001 57.565001) (width 0.25) (layer F.Cu) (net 10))
 (segment (start 157.875001 64.594999) (end 157.8 64.67) (width 0.25) (layer F.Cu) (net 10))
 (segment (start 156.15 57.49) (end 157.8 57.49) (width 0.25) (layer F.Cu) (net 10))
 (segment (start 156.064 57.404) (end 156.15 57.49) (width 0.25) (layer F.Cu) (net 10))
 (segment (start 154.0002 57.2389) (end 155.8989 57.2389) (width 0.25) (layer F.Cu) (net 10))
 (segment (start 155.8989 57.2389) (end 156.15 57.49) (width 0.25) (layer F.Cu) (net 10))
 (via (at 154.0002 57.2389) (size 0.8) (drill 0.4) (layers F.Cu B.Cu) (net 10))
 (segment (start 154.400199 59.554801) (end 154.055 59.9) (width 0.25) (layer B.Cu) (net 10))
 (segment (start 154.400199 57.638899) (end 154.400199 59.554801) (width 0.25) (layer B.Cu) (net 10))
 (segment (start 154.0002 57.2389) (end 154.400199 57.638899) (width 0.25) (layer B.Cu) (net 10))
 (segment (start 152.105 67.592998) (end 152.30499 67.792988) (width 0.25) (layer B.Cu) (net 6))
 (segment (start 152.30499 67.792988) (end 152.30499 68.59899) (width 0.25) (layer B.Cu) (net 6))
 (segment (start 152.30499 68.59899) (end 153.175 69.469) (width 0.25) (layer B.Cu) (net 6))
 (segment (start 156.1028 69.0372) (end 156.15 68.99) (width 0.25) (layer F.Cu) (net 3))
 (segment (start 153.074 61.81) (end 151.13 63.754) (width 0.25) (layer F.Cu) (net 3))
 (segment (start 156.15 61.81) (end 153.074 61.81) (width 0.25) (layer F.Cu) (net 3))
 (segment (start 157.8 68.99) (end 156.15 68.99) (width 0.25) (layer F.Cu) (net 3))
 (segment (start 157.875001 69.065001) (end 157.8 68.99) (width 0.25) (layer F.Cu) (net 3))
 (segment (start 157.810001 71.205001) (end 157.875001 71.140001) (width 0.25) (layer F.Cu) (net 3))
 (segment (start 150.453001 71.205001) (end 157.810001 71.205001) (width 0.25) (layer F.Cu) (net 3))
 (segment (start 149.634501 70.386501) (end 150.453001 71.205001) (width 0.25) (layer F.Cu) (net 3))
 (segment (start 149.634501 65.249499) (end 149.634501 70.386501) (width 0.25) (layer F.Cu) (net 3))
 (segment (start 157.875001 71.140001) (end 157.875001 69.065001) (width 0.25) (layer F.Cu) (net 3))
 (segment (start 151.13 63.754) (end 149.634501 65.249499) (width 0.25) (layer F.Cu) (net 3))
 (segment (start 149.505 66.3625) (end 149.505 65.379) (width 0.25) (layer B.Cu) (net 3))
 (segment (start 149.505 65.379) (end 151.13 63.754) (width 0.25) (layer B.Cu) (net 3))
 (via (at 151.13 63.754) (size 0.8) (drill 0.4) (layers F.Cu B.Cu) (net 3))
 (segment (start 149.505 66.3625) (end 149.505 67.1) (width 0.25) (layer B.Cu) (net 3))
 (segment (start 156.1393 58.9407) (end 156.15 58.93) (width 0.25) (layer F.Cu) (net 11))
 (segment (start 156.148 58.928) (end 156.15 58.93) (width 0.25) (layer F.Cu) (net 11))
 (segment (start 154.053 58.93) (end 153.543 58.42) (width 0.25) (layer F.Cu) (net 11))
 (segment (start 156.15 58.93) (end 154.053 58.93) (width 0.25) (layer F.Cu) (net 11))
 (segment (start 157.8 66.11) (end 156.15 66.11) (width 0.25) (layer F.Cu) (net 11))
 (segment (start 158.32501 65.58499) (end 157.8 66.11) (width 0.25) (layer F.Cu) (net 11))
 (segment (start 158.32501 57.230008) (end 158.32501 65.58499) (width 0.25) (layer F.Cu) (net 11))
 (segment (start 157.608901 56.513899) (end 158.32501 57.230008) (width 0.25) (layer F.Cu) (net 11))
 (segment (start 153.652199 56.513899) (end 157.608901 56.513899) (width 0.25) (layer F.Cu) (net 11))
 (segment (start 153.143001 57.023097) (end 153.652199 56.513899) (width 0.25) (layer F.Cu) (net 11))
 (segment (start 153.143001 58.020001) (end 153.143001 57.023097) (width 0.25) (layer F.Cu) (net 11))
 (segment (start 153.543 58.42) (end 153.143001 58.020001) (width 0.25) (layer F.Cu) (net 11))
 (via (at 153.543 58.42) (size 0.8) (drill 0.4) (layers F.Cu B.Cu) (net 11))
 (segment (start 153.405 58.558) (end 153.405 59.9) (width 0.25) (layer B.Cu) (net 11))
 (segment (start 153.543 58.42) (end 153.405 58.558) (width 0.25) (layer B.Cu) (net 11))
 (segment (start 149.505 57.697) (end 149.505 59.9) (width 0.25) (layer B.Cu) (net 16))
 (segment (start 149.212 57.404) (end 149.505 57.697) (width 0.25) (layer B.Cu) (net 16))
 (segment (start 152.105 59.264998) (end 152.105 59.9) (width 0.25) (layer B.Cu) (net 13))
 (segment (start 152.5 58.869998) (end 152.105 59.264998) (width 0.25) (layer B.Cu) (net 13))
 (segment (start 152.5 57.889166) (end 152.5 58.869998) (width 0.25) (layer B.Cu) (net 13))
 (segment (start 151.214824 56.60399) (end 152.5 57.889166) (width 0.25) (layer B.Cu) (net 13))
 (segment (start 146.89601 56.60399) (end 151.214824 56.60399) (width 0.25) (layer B.Cu) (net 13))
 (segment (start 146.192 57.308) (end 146.89601 56.60399) (width 0.25) (layer B.Cu) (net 13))
 (segment (start 146.192 59.5) (end 146.192 57.308) (width 0.25) (layer B.Cu) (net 13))
 (segment (start 150.155 61.522102) (end 150.155 59.9) (width 0.25) (layer B.Cu) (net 15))
 (segment (start 149.198102 62.479) (end 150.155 61.522102) (width 0.25) (layer B.Cu) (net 15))
 (segment (start 146.192 62.479) (end 149.198102 62.479) (width 0.25) (layer B.Cu) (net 15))
 (segment (start 148.368011 71.279011) (end 147.801599 71.279011) (width 0.25) (layer B.Cu) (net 8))
 (segment (start 148.684989 71.279011) (end 148.368011 71.279011) (width 0.25) (layer B.Cu) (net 8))
 (segment (start 153.405 67.809756) (end 154.40002 68.804776) (width 0.25) (layer B.Cu) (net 8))
 (segment (start 154.40002 68.804776) (end 154.400019 70.133225) (width 0.25) (layer B.Cu) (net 8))
 (segment (start 154.400019 70.133225) (end 153.254233 71.279011) (width 0.25) (layer B.Cu) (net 8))
 (segment (start 153.405 67.809756) (end 153.405 67.1) (width 0.25) (layer B.Cu) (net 8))
 (via (at 151.257 68.326) (size 0.8) (drill 0.4) (layers F.Cu B.Cu) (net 20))
 (segment (start 151.511 69.355) (end 151.625 69.469) (width 0.25) (layer B.Cu) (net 20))
 (segment (start 151.257 69.101) (end 151.625 69.469) (width 0.25) (layer B.Cu) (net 20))
 (segment (start 151.257 68.326) (end 151.257 69.101) (width 0.25) (layer B.Cu) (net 20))
 (segment (start 152.033 67.55) (end 156.15 67.55) (width 0.25) (layer F.Cu) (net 20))
 (segment (start 151.257 68.326) (end 152.033 67.55) (width 0.25) (layer F.Cu) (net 20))
 (via (at 151.765 58.42) (size 0.8) (drill 0.4) (layers F.Cu B.Cu) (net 21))
 (segment (start 153.715 60.37) (end 151.765 58.42) (width 0.25) (layer F.Cu) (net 21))
 (segment (start 156.15 60.37) (end 153.715 60.37) (width 0.25) (layer F.Cu) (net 21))
 (segment (start 150.762 57.417) (end 151.765 58.42) (width 0.25) (layer B.Cu) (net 21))
 (segment (start 150.762 57.404) (end 150.762 57.417) (width 0.25) (layer B.Cu) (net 21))
 (segment (start 152.755 67.796166) (end 152.755 67.1) (width 0.25) (layer B.Cu) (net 7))
 (segment (start 153.95001 68.991176) (end 152.755 67.796166) (width 0.25) (layer B.Cu) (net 7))
 (segment (start 153.95001 69.946824) (end 153.95001 68.991176) (width 0.25) (layer B.Cu) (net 7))
 (segment (start 153.067833 70.829001) (end 153.95001 69.946824) (width 0.25) (layer B.Cu) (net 7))
 (segment (start 147.160989 70.160989) (end 147.829001 70.829001) (width 0.25) (layer B.Cu) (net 7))
 (segment (start 147.160989 66.426989) (end 147.160989 70.160989) (width 0.25) (layer B.Cu) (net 7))
 (segment (start 147.829001 70.829001) (end 153.067833 70.829001) (width 0.25) (layer B.Cu) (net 7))
 (segment (start 146.192 65.458) (end 147.160989 66.426989) (width 0.25) (layer B.Cu) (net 7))
 (segment (start 147.642601 71.279011) (end 149.220989 71.279011) (width 0.25) (layer B.Cu) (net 8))
 (segment (start 146.192 69.82841) (end 147.642601 71.279011) (width 0.25) (layer B.Cu) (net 8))
 (segment (start 146.192 68.437) (end 146.192 69.82841) (width 0.25) (layer B.Cu) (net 8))
 (segment (start 149.220989 71.279011) (end 148.684989 71.279011) (width 0.25) (layer B.Cu) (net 8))
 (segment (start 153.254233 71.279011) (end 149.220989 71.279011) (width 0.25) (layer B.Cu) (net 8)))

